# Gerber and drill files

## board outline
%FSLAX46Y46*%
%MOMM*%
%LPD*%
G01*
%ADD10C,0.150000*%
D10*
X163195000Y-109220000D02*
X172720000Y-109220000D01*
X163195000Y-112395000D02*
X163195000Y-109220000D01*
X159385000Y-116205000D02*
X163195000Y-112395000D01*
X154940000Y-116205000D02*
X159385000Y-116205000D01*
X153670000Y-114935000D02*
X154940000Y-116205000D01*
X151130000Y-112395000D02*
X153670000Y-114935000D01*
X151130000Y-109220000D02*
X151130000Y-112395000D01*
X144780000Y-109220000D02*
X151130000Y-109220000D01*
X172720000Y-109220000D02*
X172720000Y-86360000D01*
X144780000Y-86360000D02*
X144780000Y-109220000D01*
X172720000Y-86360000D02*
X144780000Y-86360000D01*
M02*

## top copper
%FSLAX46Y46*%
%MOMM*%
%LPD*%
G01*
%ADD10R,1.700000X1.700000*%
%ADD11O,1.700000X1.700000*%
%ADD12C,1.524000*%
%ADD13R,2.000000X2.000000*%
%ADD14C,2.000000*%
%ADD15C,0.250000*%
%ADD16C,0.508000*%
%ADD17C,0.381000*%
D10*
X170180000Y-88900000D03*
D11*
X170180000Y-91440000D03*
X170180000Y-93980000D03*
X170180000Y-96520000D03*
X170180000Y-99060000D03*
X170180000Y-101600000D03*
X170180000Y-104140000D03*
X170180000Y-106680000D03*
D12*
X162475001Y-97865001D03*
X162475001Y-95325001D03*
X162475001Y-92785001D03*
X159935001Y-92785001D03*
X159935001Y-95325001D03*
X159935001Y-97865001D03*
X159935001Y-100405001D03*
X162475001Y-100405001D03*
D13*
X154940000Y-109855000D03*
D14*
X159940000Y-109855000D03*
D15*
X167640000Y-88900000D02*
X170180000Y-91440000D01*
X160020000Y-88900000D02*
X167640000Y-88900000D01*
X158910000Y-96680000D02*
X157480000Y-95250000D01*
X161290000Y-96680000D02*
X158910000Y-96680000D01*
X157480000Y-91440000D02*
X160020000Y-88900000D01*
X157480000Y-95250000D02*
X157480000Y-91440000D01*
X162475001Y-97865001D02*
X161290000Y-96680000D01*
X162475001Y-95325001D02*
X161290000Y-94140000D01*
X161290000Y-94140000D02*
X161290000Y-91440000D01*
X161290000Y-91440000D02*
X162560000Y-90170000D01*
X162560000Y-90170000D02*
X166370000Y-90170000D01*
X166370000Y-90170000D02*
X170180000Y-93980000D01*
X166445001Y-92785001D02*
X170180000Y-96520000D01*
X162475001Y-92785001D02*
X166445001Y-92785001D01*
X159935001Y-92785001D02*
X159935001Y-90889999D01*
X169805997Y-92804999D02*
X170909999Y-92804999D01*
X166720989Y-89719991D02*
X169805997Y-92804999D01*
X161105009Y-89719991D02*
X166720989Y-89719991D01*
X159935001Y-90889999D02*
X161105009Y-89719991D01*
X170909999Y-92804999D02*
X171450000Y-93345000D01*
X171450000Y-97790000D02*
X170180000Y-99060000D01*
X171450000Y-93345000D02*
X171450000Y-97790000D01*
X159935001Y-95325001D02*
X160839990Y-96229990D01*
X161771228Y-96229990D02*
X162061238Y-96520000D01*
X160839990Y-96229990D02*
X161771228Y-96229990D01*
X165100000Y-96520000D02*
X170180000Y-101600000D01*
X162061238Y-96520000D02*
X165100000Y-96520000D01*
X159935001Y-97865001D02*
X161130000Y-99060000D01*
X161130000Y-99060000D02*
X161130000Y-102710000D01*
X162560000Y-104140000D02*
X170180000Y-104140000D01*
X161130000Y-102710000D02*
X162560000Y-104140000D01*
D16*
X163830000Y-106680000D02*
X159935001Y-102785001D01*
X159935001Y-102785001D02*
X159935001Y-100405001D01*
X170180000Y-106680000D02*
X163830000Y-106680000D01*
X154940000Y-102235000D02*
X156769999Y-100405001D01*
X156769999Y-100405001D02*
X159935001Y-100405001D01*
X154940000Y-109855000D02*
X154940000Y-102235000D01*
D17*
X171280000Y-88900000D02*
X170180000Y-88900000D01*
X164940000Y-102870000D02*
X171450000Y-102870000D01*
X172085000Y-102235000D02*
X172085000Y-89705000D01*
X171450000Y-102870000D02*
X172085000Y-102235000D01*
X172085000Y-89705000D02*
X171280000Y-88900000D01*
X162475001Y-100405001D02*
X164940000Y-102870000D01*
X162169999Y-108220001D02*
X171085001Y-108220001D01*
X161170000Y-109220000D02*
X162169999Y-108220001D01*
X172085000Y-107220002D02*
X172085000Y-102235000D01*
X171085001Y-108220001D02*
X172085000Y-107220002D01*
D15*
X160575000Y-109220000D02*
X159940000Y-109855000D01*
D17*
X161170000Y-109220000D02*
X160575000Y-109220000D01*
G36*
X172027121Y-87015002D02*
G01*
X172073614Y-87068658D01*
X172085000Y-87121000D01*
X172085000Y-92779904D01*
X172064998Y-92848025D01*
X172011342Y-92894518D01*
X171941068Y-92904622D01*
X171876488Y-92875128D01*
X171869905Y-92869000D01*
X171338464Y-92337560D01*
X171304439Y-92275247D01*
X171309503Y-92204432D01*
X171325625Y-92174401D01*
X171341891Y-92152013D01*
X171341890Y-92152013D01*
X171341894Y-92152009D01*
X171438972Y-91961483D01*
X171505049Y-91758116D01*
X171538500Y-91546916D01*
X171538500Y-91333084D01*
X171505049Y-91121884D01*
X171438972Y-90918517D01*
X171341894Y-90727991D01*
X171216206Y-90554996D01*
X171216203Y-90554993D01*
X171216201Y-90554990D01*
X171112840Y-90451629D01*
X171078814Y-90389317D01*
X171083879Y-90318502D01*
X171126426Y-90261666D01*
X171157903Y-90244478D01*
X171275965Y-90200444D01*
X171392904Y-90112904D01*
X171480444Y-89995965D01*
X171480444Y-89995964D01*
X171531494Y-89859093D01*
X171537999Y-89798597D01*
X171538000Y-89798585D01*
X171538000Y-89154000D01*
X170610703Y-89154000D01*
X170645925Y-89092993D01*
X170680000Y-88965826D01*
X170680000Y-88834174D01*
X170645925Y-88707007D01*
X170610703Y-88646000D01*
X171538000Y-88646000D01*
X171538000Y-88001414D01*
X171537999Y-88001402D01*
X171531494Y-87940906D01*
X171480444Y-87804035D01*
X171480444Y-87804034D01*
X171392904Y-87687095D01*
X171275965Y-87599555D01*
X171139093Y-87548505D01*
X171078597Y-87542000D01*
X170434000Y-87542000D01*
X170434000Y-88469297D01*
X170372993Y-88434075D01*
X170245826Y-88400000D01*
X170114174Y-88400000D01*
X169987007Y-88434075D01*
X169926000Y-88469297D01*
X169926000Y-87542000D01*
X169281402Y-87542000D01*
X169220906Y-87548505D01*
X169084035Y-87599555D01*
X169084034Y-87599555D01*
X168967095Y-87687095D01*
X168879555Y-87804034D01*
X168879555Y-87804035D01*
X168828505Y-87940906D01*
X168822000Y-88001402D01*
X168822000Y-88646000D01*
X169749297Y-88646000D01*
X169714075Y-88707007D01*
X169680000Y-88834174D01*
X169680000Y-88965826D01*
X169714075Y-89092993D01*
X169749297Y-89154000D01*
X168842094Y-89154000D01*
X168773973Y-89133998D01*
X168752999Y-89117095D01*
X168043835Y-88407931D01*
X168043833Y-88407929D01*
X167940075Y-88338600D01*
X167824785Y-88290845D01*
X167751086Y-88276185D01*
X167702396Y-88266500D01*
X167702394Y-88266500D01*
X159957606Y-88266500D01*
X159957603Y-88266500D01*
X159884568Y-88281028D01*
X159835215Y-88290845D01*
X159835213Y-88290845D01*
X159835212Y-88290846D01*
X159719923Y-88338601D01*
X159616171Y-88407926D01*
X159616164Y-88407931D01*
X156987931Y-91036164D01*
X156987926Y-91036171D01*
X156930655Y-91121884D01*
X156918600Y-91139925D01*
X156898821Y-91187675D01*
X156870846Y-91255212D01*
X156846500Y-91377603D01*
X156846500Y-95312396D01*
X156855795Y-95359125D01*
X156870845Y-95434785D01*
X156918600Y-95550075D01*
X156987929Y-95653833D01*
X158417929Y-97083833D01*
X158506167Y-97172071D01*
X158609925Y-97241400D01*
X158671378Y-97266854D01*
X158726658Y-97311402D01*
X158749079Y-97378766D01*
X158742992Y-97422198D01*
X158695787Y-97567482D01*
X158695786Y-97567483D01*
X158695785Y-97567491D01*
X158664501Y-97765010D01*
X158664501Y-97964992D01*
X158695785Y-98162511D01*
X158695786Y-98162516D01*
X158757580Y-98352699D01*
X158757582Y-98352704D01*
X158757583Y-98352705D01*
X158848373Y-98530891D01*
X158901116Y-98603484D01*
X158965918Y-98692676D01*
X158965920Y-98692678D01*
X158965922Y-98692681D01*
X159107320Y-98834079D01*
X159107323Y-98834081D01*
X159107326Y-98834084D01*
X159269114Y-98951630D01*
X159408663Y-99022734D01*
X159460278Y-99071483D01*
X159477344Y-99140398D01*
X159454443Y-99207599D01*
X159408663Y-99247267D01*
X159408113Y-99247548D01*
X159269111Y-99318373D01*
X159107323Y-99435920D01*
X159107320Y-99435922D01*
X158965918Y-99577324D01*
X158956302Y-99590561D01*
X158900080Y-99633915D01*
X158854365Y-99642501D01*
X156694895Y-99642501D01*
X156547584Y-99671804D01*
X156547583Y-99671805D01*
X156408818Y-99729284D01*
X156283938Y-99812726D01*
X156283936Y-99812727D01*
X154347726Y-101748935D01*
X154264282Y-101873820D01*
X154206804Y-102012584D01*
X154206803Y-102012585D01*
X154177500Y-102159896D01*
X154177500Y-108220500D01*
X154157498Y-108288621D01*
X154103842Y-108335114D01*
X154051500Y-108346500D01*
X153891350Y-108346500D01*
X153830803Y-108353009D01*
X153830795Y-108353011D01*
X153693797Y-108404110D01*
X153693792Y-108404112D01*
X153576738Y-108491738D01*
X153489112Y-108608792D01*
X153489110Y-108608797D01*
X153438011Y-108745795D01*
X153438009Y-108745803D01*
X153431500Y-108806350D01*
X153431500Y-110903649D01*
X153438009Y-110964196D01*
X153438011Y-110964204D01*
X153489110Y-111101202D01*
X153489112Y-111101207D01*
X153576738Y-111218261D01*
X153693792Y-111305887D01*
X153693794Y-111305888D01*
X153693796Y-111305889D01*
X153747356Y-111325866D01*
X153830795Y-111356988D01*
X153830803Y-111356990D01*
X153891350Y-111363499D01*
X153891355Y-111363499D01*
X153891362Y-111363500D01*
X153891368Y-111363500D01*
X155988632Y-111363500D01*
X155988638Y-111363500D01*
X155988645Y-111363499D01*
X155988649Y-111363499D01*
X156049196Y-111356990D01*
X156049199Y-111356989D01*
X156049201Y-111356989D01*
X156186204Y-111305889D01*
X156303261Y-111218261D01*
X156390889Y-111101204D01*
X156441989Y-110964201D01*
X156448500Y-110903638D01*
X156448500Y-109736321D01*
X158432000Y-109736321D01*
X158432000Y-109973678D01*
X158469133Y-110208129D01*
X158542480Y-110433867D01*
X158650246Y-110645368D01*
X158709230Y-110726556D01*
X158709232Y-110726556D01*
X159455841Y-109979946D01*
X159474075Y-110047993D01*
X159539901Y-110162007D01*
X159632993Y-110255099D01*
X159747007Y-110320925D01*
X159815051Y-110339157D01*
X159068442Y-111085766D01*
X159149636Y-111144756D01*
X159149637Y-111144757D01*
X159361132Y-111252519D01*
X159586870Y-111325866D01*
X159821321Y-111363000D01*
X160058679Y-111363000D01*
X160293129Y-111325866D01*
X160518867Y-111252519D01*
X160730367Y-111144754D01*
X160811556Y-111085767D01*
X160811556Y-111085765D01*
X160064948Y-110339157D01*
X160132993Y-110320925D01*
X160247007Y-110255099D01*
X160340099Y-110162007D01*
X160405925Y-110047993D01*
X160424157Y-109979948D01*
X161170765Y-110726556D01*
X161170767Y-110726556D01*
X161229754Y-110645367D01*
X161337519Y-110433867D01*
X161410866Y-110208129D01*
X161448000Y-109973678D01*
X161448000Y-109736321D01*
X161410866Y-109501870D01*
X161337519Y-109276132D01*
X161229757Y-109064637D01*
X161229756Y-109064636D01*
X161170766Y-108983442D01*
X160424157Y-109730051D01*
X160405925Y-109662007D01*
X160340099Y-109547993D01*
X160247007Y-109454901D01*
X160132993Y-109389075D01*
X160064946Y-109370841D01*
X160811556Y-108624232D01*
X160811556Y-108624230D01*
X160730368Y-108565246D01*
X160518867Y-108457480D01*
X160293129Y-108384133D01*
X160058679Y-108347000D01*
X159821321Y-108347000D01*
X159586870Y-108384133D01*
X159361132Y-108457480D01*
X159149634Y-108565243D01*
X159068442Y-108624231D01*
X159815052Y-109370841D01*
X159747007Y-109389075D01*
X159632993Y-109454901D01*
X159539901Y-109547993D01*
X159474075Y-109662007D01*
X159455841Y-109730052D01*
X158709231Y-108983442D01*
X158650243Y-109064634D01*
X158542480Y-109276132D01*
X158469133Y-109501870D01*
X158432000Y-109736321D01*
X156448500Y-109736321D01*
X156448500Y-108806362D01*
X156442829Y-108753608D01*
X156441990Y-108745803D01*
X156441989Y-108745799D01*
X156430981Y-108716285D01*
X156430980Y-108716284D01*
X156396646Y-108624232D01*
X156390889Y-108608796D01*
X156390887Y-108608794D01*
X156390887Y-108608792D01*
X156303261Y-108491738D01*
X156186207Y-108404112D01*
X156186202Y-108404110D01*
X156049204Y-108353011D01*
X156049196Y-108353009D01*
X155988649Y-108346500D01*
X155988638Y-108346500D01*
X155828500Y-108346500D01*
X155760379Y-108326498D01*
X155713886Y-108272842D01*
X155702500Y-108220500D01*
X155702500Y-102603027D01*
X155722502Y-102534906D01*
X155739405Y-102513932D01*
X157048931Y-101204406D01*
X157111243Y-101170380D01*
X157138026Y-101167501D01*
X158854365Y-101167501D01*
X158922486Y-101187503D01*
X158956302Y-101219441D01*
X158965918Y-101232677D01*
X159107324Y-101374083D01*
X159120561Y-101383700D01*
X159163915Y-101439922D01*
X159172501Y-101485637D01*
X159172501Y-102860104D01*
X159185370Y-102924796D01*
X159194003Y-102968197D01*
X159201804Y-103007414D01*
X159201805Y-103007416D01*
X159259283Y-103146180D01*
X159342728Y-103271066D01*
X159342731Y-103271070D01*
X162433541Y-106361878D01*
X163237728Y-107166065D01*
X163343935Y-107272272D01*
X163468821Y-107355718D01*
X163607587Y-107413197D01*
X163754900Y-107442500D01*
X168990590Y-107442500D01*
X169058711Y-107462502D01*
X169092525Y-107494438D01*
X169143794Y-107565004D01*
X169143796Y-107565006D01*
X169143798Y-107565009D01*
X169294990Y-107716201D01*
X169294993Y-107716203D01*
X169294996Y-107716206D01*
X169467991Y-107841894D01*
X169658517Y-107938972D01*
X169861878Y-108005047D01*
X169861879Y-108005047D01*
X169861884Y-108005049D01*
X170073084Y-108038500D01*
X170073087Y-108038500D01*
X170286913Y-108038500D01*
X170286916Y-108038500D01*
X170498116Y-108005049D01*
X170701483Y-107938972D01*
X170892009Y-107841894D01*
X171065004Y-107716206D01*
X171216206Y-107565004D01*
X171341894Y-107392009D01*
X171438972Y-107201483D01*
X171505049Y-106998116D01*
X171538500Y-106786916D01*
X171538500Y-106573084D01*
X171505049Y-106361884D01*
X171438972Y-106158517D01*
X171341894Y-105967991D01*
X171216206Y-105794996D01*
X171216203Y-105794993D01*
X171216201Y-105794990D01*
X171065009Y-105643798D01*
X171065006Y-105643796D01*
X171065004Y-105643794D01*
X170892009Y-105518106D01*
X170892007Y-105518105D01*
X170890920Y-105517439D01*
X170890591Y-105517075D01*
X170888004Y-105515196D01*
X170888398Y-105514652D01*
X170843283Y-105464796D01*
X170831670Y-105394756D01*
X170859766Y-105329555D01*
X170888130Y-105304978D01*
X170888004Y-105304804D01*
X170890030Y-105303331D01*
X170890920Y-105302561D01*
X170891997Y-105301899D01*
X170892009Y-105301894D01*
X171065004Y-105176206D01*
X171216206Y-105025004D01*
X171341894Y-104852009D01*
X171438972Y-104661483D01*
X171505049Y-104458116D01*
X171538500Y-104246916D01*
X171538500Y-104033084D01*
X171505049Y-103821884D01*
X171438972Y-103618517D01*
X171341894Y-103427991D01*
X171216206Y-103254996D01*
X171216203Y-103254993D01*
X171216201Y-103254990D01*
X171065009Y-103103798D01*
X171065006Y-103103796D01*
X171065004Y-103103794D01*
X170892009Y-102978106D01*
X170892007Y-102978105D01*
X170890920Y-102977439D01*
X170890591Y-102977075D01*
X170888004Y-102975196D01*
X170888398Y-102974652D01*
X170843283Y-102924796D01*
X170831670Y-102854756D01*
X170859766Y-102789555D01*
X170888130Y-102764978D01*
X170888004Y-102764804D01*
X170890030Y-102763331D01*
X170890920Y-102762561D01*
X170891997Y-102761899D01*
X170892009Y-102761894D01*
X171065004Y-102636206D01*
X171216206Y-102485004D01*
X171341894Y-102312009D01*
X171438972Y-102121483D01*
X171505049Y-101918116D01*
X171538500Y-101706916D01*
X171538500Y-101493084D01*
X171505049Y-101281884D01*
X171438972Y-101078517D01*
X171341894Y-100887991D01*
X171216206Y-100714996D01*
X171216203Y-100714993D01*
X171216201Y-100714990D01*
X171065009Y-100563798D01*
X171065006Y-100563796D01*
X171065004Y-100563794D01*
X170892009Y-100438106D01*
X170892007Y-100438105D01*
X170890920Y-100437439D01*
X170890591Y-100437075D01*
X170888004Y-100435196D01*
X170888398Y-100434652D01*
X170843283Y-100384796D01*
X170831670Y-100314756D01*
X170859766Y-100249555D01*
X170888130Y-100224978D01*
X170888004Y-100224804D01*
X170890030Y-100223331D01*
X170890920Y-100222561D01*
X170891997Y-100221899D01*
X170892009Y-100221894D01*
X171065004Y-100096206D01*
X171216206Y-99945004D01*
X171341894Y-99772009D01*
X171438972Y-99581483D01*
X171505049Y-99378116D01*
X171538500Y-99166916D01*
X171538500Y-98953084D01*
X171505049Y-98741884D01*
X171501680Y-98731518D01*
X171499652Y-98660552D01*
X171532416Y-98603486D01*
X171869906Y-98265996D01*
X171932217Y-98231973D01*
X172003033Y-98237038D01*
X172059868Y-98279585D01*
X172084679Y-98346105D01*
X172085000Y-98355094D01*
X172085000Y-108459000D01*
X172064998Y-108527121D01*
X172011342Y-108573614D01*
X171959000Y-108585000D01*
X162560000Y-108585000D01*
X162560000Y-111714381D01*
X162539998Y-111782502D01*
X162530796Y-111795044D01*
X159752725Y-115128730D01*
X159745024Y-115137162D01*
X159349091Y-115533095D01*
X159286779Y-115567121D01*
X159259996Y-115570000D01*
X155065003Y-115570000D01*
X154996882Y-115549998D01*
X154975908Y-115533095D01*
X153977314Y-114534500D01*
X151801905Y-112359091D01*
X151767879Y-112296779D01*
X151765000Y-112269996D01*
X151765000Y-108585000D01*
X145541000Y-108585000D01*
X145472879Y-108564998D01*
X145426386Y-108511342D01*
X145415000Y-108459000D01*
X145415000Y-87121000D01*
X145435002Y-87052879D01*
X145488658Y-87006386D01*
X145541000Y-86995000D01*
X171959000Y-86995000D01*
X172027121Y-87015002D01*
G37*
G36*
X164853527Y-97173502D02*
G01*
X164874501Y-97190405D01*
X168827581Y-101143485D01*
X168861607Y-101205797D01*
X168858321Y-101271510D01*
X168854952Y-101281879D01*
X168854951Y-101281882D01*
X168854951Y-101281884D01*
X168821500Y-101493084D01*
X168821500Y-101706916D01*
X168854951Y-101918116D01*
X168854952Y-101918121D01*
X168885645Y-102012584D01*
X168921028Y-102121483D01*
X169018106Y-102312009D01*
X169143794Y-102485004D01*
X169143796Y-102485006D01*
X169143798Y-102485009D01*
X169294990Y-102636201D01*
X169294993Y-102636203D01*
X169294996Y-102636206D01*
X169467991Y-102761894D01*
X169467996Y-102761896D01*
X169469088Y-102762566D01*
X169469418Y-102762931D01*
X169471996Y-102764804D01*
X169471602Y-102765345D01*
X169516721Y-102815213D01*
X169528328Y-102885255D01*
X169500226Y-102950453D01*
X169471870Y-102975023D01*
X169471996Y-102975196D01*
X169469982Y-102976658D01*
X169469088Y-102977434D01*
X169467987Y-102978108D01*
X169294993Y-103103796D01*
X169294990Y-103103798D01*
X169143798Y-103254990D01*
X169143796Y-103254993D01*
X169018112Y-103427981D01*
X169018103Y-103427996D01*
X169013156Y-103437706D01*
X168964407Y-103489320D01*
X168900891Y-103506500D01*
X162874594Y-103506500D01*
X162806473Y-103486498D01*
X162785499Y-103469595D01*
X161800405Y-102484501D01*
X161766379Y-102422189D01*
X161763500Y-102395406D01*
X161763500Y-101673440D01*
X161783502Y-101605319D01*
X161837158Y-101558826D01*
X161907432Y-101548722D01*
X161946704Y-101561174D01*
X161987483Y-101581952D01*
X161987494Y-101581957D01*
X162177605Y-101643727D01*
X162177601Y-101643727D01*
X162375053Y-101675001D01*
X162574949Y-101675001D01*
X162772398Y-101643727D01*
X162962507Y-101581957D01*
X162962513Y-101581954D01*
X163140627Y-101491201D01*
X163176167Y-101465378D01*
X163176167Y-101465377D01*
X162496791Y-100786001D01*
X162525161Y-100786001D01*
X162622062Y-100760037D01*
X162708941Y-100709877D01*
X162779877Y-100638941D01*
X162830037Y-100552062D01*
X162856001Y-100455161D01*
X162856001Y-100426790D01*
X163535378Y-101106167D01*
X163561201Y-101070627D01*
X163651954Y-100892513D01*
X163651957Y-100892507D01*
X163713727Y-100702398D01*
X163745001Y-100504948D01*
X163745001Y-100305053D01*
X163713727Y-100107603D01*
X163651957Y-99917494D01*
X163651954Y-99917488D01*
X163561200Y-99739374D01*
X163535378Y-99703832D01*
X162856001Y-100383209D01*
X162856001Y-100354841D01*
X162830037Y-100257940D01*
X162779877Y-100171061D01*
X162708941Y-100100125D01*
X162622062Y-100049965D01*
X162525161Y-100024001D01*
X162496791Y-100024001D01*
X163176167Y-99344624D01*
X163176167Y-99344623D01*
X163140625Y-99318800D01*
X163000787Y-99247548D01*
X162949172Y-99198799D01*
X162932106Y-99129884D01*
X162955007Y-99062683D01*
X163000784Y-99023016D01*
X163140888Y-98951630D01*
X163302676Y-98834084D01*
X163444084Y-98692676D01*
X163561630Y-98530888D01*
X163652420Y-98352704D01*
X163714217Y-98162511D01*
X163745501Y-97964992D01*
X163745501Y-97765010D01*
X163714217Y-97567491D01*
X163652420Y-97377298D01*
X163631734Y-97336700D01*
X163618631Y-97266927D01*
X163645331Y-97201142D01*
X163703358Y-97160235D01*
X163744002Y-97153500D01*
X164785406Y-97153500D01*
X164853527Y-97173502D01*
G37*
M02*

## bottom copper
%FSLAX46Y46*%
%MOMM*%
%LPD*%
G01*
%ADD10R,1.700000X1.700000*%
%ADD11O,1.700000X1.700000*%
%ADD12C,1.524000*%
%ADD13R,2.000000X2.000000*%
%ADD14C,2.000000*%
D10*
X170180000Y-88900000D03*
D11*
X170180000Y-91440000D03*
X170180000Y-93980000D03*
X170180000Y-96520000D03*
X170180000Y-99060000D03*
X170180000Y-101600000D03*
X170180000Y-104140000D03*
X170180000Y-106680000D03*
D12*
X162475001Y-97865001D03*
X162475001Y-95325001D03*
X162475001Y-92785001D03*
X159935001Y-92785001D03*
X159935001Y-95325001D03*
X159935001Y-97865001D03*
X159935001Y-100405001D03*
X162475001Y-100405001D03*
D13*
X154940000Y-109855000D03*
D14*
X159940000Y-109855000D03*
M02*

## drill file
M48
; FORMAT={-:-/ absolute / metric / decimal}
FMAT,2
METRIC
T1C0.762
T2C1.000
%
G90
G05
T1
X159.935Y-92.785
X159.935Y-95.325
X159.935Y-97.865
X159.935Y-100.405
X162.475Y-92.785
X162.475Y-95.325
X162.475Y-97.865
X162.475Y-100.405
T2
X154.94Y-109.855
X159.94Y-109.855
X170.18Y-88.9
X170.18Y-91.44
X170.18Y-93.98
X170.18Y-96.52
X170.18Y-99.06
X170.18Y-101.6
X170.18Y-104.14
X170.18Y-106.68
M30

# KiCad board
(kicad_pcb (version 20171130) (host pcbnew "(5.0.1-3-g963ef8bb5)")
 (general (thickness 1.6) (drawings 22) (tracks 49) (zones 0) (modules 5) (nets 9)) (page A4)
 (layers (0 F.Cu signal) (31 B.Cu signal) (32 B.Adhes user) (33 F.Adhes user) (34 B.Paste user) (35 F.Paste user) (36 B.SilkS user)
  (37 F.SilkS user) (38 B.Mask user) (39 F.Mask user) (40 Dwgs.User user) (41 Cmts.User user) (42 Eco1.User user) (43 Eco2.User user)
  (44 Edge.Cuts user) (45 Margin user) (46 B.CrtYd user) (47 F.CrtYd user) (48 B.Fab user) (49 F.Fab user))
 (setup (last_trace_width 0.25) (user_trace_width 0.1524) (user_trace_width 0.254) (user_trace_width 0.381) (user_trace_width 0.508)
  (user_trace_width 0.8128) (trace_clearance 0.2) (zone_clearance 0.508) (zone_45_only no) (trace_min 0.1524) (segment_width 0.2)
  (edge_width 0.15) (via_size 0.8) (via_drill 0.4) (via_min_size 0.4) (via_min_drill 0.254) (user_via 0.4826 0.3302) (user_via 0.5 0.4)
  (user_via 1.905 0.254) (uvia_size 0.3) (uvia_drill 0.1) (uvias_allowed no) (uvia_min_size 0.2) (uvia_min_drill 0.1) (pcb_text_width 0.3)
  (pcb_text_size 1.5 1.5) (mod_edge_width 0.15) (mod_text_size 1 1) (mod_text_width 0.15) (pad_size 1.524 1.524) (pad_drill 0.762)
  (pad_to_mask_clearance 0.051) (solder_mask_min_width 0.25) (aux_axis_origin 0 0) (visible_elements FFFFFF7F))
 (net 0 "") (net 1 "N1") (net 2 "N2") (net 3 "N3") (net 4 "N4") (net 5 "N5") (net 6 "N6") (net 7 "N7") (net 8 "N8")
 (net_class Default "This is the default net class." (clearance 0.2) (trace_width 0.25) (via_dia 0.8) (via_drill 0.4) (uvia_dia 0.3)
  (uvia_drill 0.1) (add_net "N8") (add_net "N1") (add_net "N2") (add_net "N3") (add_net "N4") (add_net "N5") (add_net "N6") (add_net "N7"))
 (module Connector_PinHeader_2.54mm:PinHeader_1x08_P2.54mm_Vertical (layer F.Cu) (at 170.18 88.9)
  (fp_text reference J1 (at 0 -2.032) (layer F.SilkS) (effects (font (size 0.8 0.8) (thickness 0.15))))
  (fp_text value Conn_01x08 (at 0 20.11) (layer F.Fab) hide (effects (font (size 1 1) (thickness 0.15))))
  (pad 1 thru_hole rect (at 0 0) (size 1.7 1.7) (drill 1) (layers *.Cu *.Mask) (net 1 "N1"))
  (pad 2 thru_hole oval (at 0 2.54) (size 1.7 1.7) (drill 1) (layers *.Cu *.Mask) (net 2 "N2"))
  (pad 3 thru_hole oval (at 0 5.08) (size 1.7 1.7) (drill 1) (layers *.Cu *.Mask) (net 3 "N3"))
  (pad 4 thru_hole oval (at 0 7.62) (size 1.7 1.7) (drill 1) (layers *.Cu *.Mask) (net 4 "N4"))
  (pad 5 thru_hole oval (at 0 10.16) (size 1.7 1.7) (drill 1) (layers *.Cu *.Mask) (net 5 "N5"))
  (pad 6 thru_hole oval (at 0 12.7) (size 1.7 1.7) (drill 1) (layers *.Cu *.Mask) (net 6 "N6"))
  (pad 7 thru_hole oval (at 0 15.24) (size 1.7 1.7) (drill 1) (layers *.Cu *.Mask) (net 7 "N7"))
  (pad 8 thru_hole oval (at 0 17.78) (size 1.7 1.7) (drill 1) (layers *.Cu *.Mask) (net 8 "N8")))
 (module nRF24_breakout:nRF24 (layer F.Cu) (at 155.490001 96.595001)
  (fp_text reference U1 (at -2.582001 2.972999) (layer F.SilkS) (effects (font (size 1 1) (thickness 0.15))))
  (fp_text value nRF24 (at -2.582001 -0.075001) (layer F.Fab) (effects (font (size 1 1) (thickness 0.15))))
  (pad 1 thru_hole circle (at 6.985 1.27) (size 1.524 1.524) (drill 0.762) (layers *.Cu *.Mask) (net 2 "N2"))
  (pad 2 thru_hole circle (at 6.985 -1.27) (size 1.524 1.524) (drill 0.762) (layers *.Cu *.Mask) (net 3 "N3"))
  (pad 3 thru_hole circle (at 6.985 -3.81) (size 1.524 1.524) (drill 0.762) (layers *.Cu *.Mask) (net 4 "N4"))
  (pad 4 thru_hole circle (at 4.445 -3.81) (size 1.524 1.524) (drill 0.762) (layers *.Cu *.Mask) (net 5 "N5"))
  (pad 5 thru_hole circle (at 4.445 -1.27) (size 1.524 1.524) (drill 0.762) (layers *.Cu *.Mask) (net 6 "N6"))
  (pad 6 thru_hole circle (at 4.445 1.27) (size 1.524 1.524) (drill 0.762) (layers *.Cu *.Mask) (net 7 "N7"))
  (pad 7 thru_hole circle (at 4.445 3.81) (size 1.524 1.524) (drill 0.762) (layers *.Cu *.Mask) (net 8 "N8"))
  (pad 0 thru_hole circle (at 6.985 3.81) (size 1.524 1.524) (drill 0.762) (layers *.Cu *.Mask) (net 1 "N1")))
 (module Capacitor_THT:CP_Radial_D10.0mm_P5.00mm (layer F.Cu) (at 154.94 109.855)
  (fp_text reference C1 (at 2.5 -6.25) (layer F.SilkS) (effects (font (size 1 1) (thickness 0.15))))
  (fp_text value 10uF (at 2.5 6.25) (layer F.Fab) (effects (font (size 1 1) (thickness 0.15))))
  (pad 1 thru_hole rect (at 0 0) (size 2 2) (drill 1) (layers *.Cu *.Mask) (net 8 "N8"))
  (pad 2 thru_hole circle (at 5 0) (size 2 2) (drill 1) (layers *.Cu *.Mask) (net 1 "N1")))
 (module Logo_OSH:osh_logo (layer F.Cu) (at 147.32 88.265)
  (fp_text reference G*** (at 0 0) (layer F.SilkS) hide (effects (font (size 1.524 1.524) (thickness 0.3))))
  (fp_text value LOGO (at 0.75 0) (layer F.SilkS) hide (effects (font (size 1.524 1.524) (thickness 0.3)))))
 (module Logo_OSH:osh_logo (layer F.Cu) (at 147.32 88.265)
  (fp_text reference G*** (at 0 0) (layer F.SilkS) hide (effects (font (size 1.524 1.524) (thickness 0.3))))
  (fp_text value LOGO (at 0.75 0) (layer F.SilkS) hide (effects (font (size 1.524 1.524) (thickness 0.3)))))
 (gr_line (start 163.195 109.22) (end 172.72 109.22) (layer Edge.Cuts) (width 0.15))
 (gr_line (start 163.195 112.395) (end 163.195 109.22) (layer Edge.Cuts) (width 0.15))
 (gr_line (start 159.385 116.205) (end 163.195 112.395) (layer Edge.Cuts) (width 0.15))
 (gr_line (start 154.94 116.205) (end 159.385 116.205) (layer Edge.Cuts) (width 0.15))
 (gr_line (start 153.67 114.935) (end 154.94 116.205) (layer Edge.Cuts) (width 0.15))
 (gr_line (start 151.13 112.395) (end 153.67 114.935) (layer Edge.Cuts) (width 0.15))
 (gr_line (start 151.13 109.22) (end 151.13 112.395) (layer Edge.Cuts) (width 0.15))
 (gr_line (start 144.78 109.22) (end 151.13 109.22) (layer Edge.Cuts) (width 0.15))
 (gr_line (start 172.72 109.22) (end 172.72 86.36) (layer Edge.Cuts) (width 0.15))
 (gr_line (start 144.78 86.36) (end 144.78 109.22) (layer Edge.Cuts) (width 0.15))
 (gr_line (start 172.72 86.36) (end 144.78 86.36) (layer Edge.Cuts) (width 0.15))
 (segment (start 167.64 88.9) (end 170.18 91.44) (width 0.25) (layer F.Cu) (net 2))
 (segment (start 160.02 88.9) (end 167.64 88.9) (width 0.25) (layer F.Cu) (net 2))
 (segment (start 158.91 96.68) (end 157.48 95.25) (width 0.25) (layer F.Cu) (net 2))
 (segment (start 161.29 96.68) (end 158.91 96.68) (width 0.25) (layer F.Cu) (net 2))
 (segment (start 157.48 91.44) (end 160.02 88.9) (width 0.25) (layer F.Cu) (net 2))
 (segment (start 157.48 95.25) (end 157.48 91.44) (width 0.25) (layer F.Cu) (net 2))
 (segment (start 162.475001 97.865001) (end 161.29 96.68) (width 0.25) (layer F.Cu) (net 2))
 (segment (start 162.475001 95.325001) (end 161.29 94.14) (width 0.25) (layer F.Cu) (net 3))
 (segment (start 161.29 94.14) (end 161.29 91.44) (width 0.25) (layer F.Cu) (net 3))
 (segment (start 161.29 91.44) (end 162.56 90.17) (width 0.25) (layer F.Cu) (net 3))
 (segment (start 162.56 90.17) (end 166.37 90.17) (width 0.25) (layer F.Cu) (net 3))
 (segment (start 166.37 90.17) (end 170.18 93.98) (width 0.25) (layer F.Cu) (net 3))
 (segment (start 166.445001 92.785001) (end 170.18 96.52) (width 0.25) (layer F.Cu) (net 4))
 (segment (start 162.475001 92.785001) (end 166.445001 92.785001) (width 0.25) (layer F.Cu) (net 4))
 (segment (start 159.935001 92.785001) (end 159.935001 90.889999) (width 0.25) (layer F.Cu) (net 5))
 (segment (start 169.805997 92.804999) (end 170.909999 92.804999) (width 0.25) (layer F.Cu) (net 5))
 (segment (start 166.720989 89.719991) (end 169.805997 92.804999) (width 0.25) (layer F.Cu) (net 5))
 (segment (start 161.105009 89.719991) (end 166.720989 89.719991) (width 0.25) (layer F.Cu) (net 5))
 (segment (start 159.935001 90.889999) (end 161.105009 89.719991) (width 0.25) (layer F.Cu) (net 5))
 (segment (start 170.909999 92.804999) (end 171.45 93.345) (width 0.25) (layer F.Cu) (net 5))
 (segment (start 171.45 97.79) (end 170.18 99.06) (width 0.25) (layer F.Cu) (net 5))
 (segment (start 171.45 93.345) (end 171.45 97.79) (width 0.25) (layer F.Cu) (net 5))
 (segment (start 159.935001 95.325001) (end 160.83999 96.22999) (width 0.25) (layer F.Cu) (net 6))
 (segment (start 161.771228 96.22999) (end 162.061238 96.52) (width 0.25) (layer F.Cu) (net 6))
 (segment (start 160.83999 96.22999) (end 161.771228 96.22999) (width 0.25) (layer F.Cu) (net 6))
 (segment (start 165.1 96.52) (end 170.18 101.6) (width 0.25) (layer F.Cu) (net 6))
 (segment (start 162.061238 96.52) (end 165.1 96.52) (width 0.25) (layer F.Cu) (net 6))
 (segment (start 159.935001 97.865001) (end 161.13 99.06) (width 0.25) (layer F.Cu) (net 7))
 (segment (start 161.13 99.06) (end 161.13 102.71) (width 0.25) (layer F.Cu) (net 7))
 (segment (start 162.56 104.14) (end 170.18 104.14) (width 0.25) (layer F.Cu) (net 7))
 (segment (start 161.13 102.71) (end 162.56 104.14) (width 0.25) (layer F.Cu) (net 7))
 (segment (start 163.83 106.68) (end 159.935001 102.785001) (width 0.508) (layer F.Cu) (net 8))
 (segment (start 159.935001 102.785001) (end 159.935001 100.405001) (width 0.508) (layer F.Cu) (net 8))
 (segment (start 170.18 106.68) (end 163.83 106.68) (width 0.508) (layer F.Cu) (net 8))
 (segment (start 154.94 102.235) (end 156.769999 100.405001) (width 0.508) (layer F.Cu) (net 8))
 (segment (start 156.769999 100.405001) (end 159.935001 100.405001) (width 0.508) (layer F.Cu) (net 8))
 (segment (start 154.94 109.855) (end 154.94 102.235) (width 0.508) (layer F.Cu) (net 8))
 (segment (start 171.28 88.9) (end 170.18 88.9) (width 0.381) (layer F.Cu) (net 1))
 (segment (start 164.94 102.87) (end 171.45 102.87) (width 0.381) (layer F.Cu) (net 1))
 (segment (start 172.085 102.235) (end 172.085 89.705) (width 0.381) (layer F.Cu) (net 1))
 (segment (start 171.45 102.87) (end 172.085 102.235) (width 0.381) (layer F.Cu) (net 1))
 (segment (start 172.085 89.705) (end 171.28 88.9) (width 0.381) (layer F.Cu) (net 1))
 (segment (start 162.475001 100.405001) (end 164.94 102.87) (width 0.381) (layer F.Cu) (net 1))
 (segment (start 162.169999 108.220001) (end 171.085001 108.220001) (width 0.381) (layer F.Cu) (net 1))
 (segment (start 161.17 109.22) (end 162.169999 108.220001) (width 0.381) (layer F.Cu) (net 1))
 (segment (start 172.085 107.220002) (end 172.085 102.235) (width 0.381) (layer F.Cu) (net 1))
 (segment (start 171.085001 108.220001) (end 172.085 107.220002) (width 0.381) (layer F.Cu) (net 1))
 (segment (start 160.575 109.22) (end 159.94 109.855) (width 0.25) (layer F.Cu) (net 1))
 (segment (start 161.17 109.22) (end 160.575 109.22) (width 0.381) (layer F.Cu) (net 1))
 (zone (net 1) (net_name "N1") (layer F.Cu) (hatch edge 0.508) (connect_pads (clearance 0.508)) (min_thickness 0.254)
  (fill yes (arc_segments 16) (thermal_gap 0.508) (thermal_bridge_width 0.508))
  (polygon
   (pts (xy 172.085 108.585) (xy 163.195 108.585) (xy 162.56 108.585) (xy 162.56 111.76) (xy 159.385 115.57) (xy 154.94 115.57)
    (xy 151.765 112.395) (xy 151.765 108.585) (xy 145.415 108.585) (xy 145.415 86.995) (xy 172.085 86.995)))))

